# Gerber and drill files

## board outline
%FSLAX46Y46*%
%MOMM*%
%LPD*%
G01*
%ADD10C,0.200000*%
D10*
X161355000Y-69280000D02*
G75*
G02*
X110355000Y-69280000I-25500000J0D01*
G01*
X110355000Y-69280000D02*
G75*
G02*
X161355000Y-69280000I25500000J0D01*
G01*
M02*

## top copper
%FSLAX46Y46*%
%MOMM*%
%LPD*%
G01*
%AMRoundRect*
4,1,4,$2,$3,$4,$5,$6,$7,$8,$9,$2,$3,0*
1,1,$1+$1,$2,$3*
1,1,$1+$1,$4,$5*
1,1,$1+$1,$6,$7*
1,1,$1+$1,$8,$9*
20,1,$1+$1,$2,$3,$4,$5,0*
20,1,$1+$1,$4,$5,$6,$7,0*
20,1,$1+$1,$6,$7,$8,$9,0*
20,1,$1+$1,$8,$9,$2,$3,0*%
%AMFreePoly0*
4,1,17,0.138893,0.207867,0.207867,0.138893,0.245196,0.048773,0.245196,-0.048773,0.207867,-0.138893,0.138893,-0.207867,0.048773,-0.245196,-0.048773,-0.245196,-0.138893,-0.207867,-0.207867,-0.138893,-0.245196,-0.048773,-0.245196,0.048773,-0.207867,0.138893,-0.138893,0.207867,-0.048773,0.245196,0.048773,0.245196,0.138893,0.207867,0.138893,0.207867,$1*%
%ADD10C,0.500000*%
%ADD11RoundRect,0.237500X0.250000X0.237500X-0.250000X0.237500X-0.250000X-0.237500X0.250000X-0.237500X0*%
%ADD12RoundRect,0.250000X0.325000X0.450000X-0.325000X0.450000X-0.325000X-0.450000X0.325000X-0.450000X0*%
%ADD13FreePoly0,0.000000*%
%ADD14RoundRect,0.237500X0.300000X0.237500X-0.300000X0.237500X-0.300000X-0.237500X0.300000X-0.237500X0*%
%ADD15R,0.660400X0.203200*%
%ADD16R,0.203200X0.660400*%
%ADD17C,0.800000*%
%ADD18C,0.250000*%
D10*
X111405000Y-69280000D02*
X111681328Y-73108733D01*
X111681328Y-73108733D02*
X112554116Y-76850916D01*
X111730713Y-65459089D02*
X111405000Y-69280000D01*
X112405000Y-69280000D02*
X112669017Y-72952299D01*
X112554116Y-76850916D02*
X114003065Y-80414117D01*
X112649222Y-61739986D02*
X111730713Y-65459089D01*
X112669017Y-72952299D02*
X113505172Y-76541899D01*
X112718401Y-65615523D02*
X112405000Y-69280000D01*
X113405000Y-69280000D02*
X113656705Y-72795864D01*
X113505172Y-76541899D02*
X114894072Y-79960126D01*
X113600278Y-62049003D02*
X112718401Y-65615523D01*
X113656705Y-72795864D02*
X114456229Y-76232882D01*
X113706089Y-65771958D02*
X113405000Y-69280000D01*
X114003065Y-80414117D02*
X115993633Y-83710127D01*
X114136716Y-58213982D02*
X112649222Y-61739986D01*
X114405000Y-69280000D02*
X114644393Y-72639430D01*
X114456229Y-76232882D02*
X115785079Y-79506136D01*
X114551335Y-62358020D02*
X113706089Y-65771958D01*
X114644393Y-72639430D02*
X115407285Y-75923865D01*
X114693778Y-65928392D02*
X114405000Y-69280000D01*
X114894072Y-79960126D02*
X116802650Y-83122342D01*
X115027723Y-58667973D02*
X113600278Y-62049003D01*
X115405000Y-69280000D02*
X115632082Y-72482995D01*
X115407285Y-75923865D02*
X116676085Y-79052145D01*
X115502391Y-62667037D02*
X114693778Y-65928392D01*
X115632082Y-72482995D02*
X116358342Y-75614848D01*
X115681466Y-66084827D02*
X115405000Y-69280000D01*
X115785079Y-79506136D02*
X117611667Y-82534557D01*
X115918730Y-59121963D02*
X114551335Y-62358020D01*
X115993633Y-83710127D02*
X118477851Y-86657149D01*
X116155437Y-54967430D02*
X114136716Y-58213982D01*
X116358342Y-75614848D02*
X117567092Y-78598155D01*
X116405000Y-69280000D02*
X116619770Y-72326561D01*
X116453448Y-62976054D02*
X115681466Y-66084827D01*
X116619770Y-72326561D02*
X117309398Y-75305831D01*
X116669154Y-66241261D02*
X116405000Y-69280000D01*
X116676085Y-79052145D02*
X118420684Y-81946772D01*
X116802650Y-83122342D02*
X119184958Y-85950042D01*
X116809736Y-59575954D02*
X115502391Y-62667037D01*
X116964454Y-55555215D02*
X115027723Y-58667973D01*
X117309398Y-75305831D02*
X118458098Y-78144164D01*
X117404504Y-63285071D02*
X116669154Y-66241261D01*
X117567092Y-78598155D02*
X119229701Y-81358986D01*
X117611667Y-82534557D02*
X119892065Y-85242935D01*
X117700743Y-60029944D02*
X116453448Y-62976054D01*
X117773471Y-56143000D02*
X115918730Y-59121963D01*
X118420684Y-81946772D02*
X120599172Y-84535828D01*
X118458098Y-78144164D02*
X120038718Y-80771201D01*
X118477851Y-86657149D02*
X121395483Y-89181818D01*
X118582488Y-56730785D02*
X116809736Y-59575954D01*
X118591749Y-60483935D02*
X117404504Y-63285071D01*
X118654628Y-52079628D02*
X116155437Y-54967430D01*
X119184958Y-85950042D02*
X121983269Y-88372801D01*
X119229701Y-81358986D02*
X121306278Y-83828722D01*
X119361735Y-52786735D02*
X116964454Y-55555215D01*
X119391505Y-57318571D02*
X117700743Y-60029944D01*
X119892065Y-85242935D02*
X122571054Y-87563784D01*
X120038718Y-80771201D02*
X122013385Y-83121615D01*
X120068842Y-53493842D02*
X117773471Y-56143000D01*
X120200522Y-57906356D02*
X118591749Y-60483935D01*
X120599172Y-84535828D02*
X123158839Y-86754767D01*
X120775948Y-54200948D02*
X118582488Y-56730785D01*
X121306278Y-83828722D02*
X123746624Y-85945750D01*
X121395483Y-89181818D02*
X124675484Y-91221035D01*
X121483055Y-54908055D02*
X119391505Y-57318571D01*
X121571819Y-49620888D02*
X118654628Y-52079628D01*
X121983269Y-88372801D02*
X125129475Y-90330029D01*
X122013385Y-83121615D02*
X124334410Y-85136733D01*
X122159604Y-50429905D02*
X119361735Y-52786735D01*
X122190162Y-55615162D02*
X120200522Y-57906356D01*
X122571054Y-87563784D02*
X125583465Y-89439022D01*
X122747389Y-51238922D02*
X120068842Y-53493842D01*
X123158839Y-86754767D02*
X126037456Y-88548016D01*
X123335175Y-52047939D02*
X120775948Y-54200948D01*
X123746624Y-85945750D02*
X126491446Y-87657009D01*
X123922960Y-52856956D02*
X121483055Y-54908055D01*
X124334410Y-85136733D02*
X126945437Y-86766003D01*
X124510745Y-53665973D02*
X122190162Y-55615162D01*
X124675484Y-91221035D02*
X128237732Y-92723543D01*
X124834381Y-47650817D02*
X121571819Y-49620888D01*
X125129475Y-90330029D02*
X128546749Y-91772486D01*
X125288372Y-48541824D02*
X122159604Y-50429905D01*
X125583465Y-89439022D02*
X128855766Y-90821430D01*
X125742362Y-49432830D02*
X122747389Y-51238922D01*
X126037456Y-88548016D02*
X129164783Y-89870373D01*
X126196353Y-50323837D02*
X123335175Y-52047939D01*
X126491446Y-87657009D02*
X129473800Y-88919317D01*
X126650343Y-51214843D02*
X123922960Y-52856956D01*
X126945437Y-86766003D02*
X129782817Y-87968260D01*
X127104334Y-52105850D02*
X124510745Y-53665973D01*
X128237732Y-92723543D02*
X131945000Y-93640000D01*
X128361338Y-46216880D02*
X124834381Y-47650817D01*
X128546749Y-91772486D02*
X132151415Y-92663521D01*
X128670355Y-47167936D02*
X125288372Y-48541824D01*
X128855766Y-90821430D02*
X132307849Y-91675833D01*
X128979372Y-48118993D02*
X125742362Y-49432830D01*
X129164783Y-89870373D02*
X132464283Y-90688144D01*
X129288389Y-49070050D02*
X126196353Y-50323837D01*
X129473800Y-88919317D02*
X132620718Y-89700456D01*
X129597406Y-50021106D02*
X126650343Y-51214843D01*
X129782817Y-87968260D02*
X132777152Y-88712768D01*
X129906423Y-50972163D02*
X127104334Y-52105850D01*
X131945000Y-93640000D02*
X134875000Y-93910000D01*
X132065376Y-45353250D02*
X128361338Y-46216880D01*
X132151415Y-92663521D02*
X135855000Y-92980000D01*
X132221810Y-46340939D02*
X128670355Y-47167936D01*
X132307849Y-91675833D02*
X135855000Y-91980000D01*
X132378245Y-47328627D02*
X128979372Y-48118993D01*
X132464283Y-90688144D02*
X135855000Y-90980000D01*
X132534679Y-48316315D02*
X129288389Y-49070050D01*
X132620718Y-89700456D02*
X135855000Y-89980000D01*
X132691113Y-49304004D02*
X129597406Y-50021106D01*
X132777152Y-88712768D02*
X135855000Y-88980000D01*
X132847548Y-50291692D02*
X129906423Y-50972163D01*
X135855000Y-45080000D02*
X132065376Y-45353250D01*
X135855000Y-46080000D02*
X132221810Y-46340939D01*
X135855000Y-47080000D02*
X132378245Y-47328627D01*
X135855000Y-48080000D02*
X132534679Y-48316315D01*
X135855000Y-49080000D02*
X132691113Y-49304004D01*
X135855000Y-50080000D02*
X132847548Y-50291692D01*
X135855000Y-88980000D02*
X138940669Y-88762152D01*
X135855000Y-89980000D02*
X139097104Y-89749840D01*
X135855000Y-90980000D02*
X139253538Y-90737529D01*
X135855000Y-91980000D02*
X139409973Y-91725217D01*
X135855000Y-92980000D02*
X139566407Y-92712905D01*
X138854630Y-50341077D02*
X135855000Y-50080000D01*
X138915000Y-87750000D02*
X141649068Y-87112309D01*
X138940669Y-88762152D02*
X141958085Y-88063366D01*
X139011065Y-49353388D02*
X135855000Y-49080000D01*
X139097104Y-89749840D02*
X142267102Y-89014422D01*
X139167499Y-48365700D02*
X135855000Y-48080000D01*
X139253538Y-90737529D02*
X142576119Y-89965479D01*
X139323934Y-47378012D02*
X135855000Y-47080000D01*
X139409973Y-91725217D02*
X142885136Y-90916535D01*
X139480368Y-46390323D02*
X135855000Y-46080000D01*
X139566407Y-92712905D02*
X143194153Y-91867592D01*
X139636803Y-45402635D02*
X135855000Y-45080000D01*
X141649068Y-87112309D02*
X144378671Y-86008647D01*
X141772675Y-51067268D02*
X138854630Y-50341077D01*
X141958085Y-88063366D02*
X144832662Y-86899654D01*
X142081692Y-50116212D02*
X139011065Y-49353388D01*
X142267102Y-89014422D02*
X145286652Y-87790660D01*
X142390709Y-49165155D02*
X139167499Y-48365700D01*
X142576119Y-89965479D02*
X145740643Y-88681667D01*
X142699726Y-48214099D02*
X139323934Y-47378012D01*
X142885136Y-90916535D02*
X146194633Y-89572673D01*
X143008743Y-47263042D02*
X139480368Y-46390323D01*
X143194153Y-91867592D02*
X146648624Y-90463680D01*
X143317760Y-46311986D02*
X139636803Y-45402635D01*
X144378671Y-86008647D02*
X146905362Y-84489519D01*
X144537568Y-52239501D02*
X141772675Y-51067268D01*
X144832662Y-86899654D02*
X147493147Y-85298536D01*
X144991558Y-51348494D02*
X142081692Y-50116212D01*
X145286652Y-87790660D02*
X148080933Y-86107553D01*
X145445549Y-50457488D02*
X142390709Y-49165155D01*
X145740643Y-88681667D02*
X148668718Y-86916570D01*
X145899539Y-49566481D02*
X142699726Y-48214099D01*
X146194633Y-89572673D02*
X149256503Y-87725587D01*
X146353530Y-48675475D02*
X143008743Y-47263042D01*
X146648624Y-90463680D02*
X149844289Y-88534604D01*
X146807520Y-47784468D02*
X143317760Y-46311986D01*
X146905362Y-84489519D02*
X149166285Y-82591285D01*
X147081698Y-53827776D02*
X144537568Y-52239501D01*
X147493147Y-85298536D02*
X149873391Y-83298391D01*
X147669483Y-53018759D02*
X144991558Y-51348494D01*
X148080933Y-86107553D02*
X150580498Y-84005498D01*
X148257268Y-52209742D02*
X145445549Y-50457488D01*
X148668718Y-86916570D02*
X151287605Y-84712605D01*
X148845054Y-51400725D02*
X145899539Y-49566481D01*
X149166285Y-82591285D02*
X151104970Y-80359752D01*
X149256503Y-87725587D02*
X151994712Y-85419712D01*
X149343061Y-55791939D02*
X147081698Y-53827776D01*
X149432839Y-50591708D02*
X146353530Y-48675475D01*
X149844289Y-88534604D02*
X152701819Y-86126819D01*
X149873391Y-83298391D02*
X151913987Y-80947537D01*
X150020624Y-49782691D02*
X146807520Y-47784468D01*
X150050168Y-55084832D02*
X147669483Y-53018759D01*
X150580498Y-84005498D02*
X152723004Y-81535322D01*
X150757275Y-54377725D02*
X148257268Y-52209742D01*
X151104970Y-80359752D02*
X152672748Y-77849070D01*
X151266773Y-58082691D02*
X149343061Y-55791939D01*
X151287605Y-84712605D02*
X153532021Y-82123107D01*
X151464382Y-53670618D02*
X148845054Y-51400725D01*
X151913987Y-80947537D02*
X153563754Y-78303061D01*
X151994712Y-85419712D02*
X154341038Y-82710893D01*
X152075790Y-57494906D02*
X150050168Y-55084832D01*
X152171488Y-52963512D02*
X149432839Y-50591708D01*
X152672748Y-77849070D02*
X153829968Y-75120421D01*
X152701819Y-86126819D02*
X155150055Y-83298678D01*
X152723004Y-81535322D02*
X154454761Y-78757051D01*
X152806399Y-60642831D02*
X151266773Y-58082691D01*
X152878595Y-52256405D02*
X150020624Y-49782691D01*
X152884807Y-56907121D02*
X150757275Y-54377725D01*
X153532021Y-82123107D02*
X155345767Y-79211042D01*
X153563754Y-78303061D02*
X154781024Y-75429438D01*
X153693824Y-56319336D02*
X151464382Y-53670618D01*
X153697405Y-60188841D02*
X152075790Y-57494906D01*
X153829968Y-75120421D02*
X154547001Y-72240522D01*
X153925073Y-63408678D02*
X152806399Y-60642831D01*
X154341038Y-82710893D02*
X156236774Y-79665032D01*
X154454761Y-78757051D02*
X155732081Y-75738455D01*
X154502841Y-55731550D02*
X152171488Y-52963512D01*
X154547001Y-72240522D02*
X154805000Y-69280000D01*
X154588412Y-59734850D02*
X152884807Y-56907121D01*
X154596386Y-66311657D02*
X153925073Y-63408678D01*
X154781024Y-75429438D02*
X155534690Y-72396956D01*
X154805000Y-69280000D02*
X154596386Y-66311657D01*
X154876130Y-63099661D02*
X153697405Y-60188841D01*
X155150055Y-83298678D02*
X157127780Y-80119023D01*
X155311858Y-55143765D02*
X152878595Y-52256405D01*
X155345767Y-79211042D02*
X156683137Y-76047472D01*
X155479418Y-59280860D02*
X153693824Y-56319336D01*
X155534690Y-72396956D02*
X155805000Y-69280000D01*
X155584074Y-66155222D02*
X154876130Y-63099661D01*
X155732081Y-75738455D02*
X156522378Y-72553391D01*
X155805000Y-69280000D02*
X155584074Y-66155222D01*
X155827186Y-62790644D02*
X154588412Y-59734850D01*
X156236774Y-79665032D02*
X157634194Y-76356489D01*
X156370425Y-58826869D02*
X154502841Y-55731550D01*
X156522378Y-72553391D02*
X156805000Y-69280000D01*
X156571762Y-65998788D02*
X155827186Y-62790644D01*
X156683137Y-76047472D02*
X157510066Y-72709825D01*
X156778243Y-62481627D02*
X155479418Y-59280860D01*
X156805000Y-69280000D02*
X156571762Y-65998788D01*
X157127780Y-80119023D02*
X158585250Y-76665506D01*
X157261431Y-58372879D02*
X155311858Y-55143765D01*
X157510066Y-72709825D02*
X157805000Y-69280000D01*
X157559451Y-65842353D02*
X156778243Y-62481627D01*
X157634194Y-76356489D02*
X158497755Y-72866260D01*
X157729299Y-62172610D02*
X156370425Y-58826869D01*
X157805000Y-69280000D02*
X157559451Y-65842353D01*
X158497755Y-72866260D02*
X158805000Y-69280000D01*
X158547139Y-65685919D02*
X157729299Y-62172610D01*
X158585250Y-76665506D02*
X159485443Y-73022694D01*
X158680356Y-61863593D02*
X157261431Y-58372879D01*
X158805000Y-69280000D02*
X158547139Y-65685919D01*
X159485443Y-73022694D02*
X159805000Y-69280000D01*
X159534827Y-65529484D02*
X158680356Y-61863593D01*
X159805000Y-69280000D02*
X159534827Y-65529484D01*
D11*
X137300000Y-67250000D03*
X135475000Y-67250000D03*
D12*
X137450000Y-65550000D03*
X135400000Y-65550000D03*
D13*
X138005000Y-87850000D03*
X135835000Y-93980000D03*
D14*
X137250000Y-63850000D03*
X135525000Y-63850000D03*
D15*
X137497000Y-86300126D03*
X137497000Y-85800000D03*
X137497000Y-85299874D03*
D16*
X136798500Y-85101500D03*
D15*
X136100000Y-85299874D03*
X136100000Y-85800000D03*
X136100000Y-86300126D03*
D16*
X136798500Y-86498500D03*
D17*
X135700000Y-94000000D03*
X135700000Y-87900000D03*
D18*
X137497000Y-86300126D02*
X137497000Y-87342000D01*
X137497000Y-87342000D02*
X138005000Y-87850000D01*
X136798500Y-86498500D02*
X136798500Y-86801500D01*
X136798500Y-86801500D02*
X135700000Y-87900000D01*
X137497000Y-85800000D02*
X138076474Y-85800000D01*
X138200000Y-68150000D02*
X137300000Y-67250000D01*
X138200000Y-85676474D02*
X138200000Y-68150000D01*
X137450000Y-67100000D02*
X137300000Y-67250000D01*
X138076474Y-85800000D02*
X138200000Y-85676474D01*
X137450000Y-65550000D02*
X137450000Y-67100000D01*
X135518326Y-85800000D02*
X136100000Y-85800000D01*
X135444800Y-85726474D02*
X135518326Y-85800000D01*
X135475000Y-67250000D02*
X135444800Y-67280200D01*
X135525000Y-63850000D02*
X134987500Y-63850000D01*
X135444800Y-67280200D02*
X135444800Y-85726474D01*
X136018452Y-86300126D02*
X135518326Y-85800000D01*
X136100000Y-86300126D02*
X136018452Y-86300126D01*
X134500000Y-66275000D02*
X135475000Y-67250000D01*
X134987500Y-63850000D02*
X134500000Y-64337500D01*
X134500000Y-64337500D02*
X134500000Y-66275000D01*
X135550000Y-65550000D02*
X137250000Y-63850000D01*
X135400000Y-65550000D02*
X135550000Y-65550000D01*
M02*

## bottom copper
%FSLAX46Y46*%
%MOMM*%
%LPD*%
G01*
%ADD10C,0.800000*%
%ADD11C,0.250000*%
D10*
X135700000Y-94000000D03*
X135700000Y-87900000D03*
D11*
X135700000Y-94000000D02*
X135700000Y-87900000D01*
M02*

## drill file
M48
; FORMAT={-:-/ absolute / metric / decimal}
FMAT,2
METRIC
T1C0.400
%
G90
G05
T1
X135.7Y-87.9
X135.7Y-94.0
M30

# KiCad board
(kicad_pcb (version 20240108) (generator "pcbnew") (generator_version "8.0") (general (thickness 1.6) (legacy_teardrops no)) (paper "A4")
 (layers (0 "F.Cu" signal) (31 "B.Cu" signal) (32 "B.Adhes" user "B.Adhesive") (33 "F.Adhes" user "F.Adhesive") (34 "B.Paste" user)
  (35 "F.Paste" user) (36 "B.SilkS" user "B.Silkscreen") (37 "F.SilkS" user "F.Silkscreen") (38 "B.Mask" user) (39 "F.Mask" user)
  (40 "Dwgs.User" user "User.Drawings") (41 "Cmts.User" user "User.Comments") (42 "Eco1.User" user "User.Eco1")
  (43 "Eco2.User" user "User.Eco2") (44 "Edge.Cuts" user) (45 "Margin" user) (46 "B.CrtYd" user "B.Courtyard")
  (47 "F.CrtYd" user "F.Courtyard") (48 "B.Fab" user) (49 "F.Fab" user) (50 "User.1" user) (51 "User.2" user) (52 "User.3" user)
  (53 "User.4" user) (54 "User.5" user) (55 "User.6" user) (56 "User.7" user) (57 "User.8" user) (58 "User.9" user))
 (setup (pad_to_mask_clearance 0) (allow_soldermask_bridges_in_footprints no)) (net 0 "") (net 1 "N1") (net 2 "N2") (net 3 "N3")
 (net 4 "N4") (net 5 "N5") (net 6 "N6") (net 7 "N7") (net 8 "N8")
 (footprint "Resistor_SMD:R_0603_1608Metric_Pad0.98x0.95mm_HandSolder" (layer "F.Cu") (at 136.3875 67.25 180)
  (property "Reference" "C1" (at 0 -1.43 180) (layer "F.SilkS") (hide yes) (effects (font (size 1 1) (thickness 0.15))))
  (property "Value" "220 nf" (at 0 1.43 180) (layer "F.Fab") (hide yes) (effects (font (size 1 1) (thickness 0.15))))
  (pad "1" smd roundrect (at -0.9125 0 180) (size 0.975 0.95) (layers "F.Cu" "F.Paste" "F.Mask") (roundrect_rratio 0.25) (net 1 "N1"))
  (pad "2" smd roundrect (at 0.9125 0 180) (size 0.975 0.95) (layers "F.Cu" "F.Paste" "F.Mask") (roundrect_rratio 0.25) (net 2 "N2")))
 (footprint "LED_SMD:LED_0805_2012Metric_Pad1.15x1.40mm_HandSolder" (layer "F.Cu") (at 136.425 65.55 180)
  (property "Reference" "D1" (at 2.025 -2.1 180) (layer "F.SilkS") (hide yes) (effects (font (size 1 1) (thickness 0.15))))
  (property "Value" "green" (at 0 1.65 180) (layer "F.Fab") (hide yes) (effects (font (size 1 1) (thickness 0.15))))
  (pad "1" smd roundrect (at -1.025 0 180) (size 1.15 1.4) (layers "F.Cu" "F.Paste" "F.Mask") (roundrect_rratio 0.2173913043) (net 1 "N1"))
  (pad "2" smd roundrect (at 1.025 0 180) (size 1.15 1.4) (layers "F.Cu" "F.Paste" "F.Mask") (roundrect_rratio 0.2173913043) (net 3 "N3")))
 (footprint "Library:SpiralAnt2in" (layer "F.Cu") (at 135.855 69.28)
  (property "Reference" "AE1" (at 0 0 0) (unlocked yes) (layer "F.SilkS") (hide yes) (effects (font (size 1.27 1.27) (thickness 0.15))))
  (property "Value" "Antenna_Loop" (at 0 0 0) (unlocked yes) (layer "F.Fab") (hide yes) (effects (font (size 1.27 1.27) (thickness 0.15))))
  (fp_line (start -24.45 0) (end -24.173672 3.828733) (stroke (width 0.5) (type default)) (layer "F.Cu"))
  (fp_line (start -24.173672 3.828733) (end -23.300884 7.570916) (stroke (width 0.5) (type default)) (layer "F.Cu"))
  (fp_line (start -24.124287 -3.820911) (end -24.45 0) (stroke (width 0.5) (type default)) (layer "F.Cu"))
  (fp_line (start -23.45 0) (end -23.185983 3.672299) (stroke (width 0.5) (type default)) (layer "F.Cu"))
  (fp_line (start -23.300884 7.570916) (end -21.851935 11.134117) (stroke (width 0.5) (type default)) (layer "F.Cu"))
  (fp_line (start -23.205778 -7.540014) (end -24.124287 -3.820911) (stroke (width 0.5) (type default)) (layer "F.Cu"))
  (fp_line (start -23.185983 3.672299) (end -22.349828 7.261899) (stroke (width 0.5) (type default)) (layer "F.Cu"))
  (fp_line (start -23.136599 -3.664477) (end -23.45 0) (stroke (width 0.5) (type default)) (layer "F.Cu"))
  (fp_line (start -22.45 0) (end -22.198295 3.515864) (stroke (width 0.5) (type default)) (layer "F.Cu"))
  (fp_line (start -22.349828 7.261899) (end -20.960928 10.680126) (stroke (width 0.5) (type default)) (layer "F.Cu"))
  (fp_line (start -22.254722 -7.230997) (end -23.136599 -3.664477) (stroke (width 0.5) (type default)) (layer "F.Cu"))
  (fp_line (start -22.198295 3.515864) (end -21.398771 6.952882) (stroke (width 0.5) (type default)) (layer "F.Cu"))
  (fp_line (start -22.148911 -3.508042) (end -22.45 0) (stroke (width 0.5) (type default)) (layer "F.Cu"))
  (fp_line (start -21.851935 11.134117) (end -19.861367 14.430127) (stroke (width 0.5) (type default)) (layer "F.Cu"))
  (fp_line (start -21.718284 -11.066018) (end -23.205778 -7.540014) (stroke (width 0.5) (type default)) (layer "F.Cu"))
  (fp_line (start -21.45 0) (end -21.210607 3.35943) (stroke (width 0.5) (type default)) (layer "F.Cu"))
  (fp_line (start -21.398771 6.952882) (end -20.069921 10.226136) (stroke (width 0.5) (type default)) (layer "F.Cu"))
  (fp_line (start -21.303665 -6.92198) (end -22.148911 -3.508042) (stroke (width 0.5) (type default)) (layer "F.Cu"))
  (fp_line (start -21.210607 3.35943) (end -20.447715 6.643865) (stroke (width 0.5) (type default)) (layer "F.Cu"))
  (fp_line (start -21.161222 -3.351608) (end -21.45 0) (stroke (width 0.5) (type default)) (layer "F.Cu"))
  (fp_line (start -20.960928 10.680126) (end -19.05235 13.842342) (stroke (width 0.5) (type default)) (layer "F.Cu"))
  (fp_line (start -20.827277 -10.612027) (end -22.254722 -7.230997) (stroke (width 0.5) (type default)) (layer "F.Cu"))
  (fp_line (start -20.45 0) (end -20.222918 3.202995) (stroke (width 0.5) (type default)) (layer "F.Cu"))
  (fp_line (start -20.447715 6.643865) (end -19.178915 9.772145) (stroke (width 0.5) (type default)) (layer "F.Cu"))
  (fp_line (start -20.352609 -6.612963) (end -21.161222 -3.351608) (stroke (width 0.5) (type default)) (layer "F.Cu"))
  (fp_line (start -20.222918 3.202995) (end -19.496658 6.334848) (stroke (width 0.5) (type default)) (layer "F.Cu"))
  (fp_line (start -20.173534 -3.195173) (end -20.45 0) (stroke (width 0.5) (type default)) (layer "F.Cu"))
  (fp_line (start -20.069921 10.226136) (end -18.243333 13.254557) (stroke (width 0.5) (type default)) (layer "F.Cu"))
  (fp_line (start -19.93627 -10.158037) (end -21.303665 -6.92198) (stroke (width 0.5) (type default)) (layer "F.Cu"))
  (fp_line (start -19.861367 14.430127) (end -17.377149 17.377149) (stroke (width 0.5) (type default)) (layer "F.Cu"))
  (fp_line (start -19.699563 -14.31257) (end -21.718284 -11.066018) (stroke (width 0.5) (type default)) (layer "F.Cu"))
  (fp_line (start -19.496658 6.334848) (end -18.287908 9.318155) (stroke (width 0.5) (type default)) (layer "F.Cu"))
  (fp_line (start -19.45 0) (end -19.23523 3.046561) (stroke (width 0.5) (type default)) (layer "F.Cu"))
  (fp_line (start -19.401552 -6.303946) (end -20.173534 -3.195173) (stroke (width 0.5) (type default)) (layer "F.Cu"))
  (fp_line (start -19.23523 3.046561) (end -18.545602 6.025831) (stroke (width 0.5) (type default)) (layer "F.Cu"))
  (fp_line (start -19.185846 -3.038739) (end -19.45 0) (stroke (width 0.5) (type default)) (layer "F.Cu"))
  (fp_line (start -19.178915 9.772145) (end -17.434316 12.666772) (stroke (width 0.5) (type default)) (layer "F.Cu"))
  (fp_line (start -19.05235 13.842342) (end -16.670042 16.670042) (stroke (width 0.5) (type default)) (layer "F.Cu"))
  (fp_line (start -19.045264 -9.704046) (end -20.352609 -6.612963) (stroke (width 0.5) (type default)) (layer "F.Cu"))
  (fp_line (start -18.890546 -13.724785) (end -20.827277 -10.612027) (stroke (width 0.5) (type default)) (layer "F.Cu"))
  (fp_line (start -18.545602 6.025831) (end -17.396902 8.864164) (stroke (width 0.5) (type default)) (layer "F.Cu"))
  (fp_line (start -18.450496 -5.994929) (end -19.185846 -3.038739) (stroke (width 0.5) (type default)) (layer "F.Cu"))
  (fp_line (start -18.287908 9.318155) (end -16.625299 12.078986) (stroke (width 0.5) (type default)) (layer "F.Cu"))
  (fp_line (start -18.243333 13.254557) (end -15.962935 15.962935) (stroke (width 0.5) (type default)) (layer "F.Cu"))
  (fp_line (start -18.154257 -9.250056) (end -19.401552 -6.303946) (stroke (width 0.5) (type default)) (layer "F.Cu"))
  (fp_line (start -18.081529 -13.137) (end -19.93627 -10.158037) (stroke (width 0.5) (type default)) (layer "F.Cu"))
  (fp_line (start -17.434316 12.666772) (end -15.255828 15.255828) (stroke (width 0.5) (type default)) (layer "F.Cu"))
  (fp_line (start -17.396902 8.864164) (end -15.816282 11.491201) (stroke (width 0.5) (type default)) (layer "F.Cu"))
  (fp_line (start -17.377149 17.377149) (end -14.459517 19.901818) (stroke (width 0.5) (type default)) (layer "F.Cu"))
  (fp_line (start -17.272512 -12.549215) (end -19.045264 -9.704046) (stroke (width 0.5) (type default)) (layer "F.Cu"))
  (fp_line (start -17.263251 -8.796065) (end -18.450496 -5.994929) (stroke (width 0.5) (type default)) (layer "F.Cu"))
  (fp_line (start -17.200372 -17.200372) (end -19.699563 -14.31257) (stroke (width 0.5) (type default)) (layer "F.Cu"))
  (fp_line (start -16.670042 16.670042) (end -13.871731 19.092801) (stroke (width 0.5) (type default)) (layer "F.Cu"))
  (fp_line (start -16.625299 12.078986) (end -14.548722 14.548722) (stroke (width 0.5) (type default)) (layer "F.Cu"))
  (fp_line (start -16.493265 -16.493265) (end -18.890546 -13.724785) (stroke (width 0.5) (type default)) (layer "F.Cu"))
  (fp_line (start -16.463495 -11.961429) (end -18.154257 -9.250056) (stroke (width 0.5) (type default)) (layer "F.Cu"))
  (fp_line (start -15.962935 15.962935) (end -13.283946 18.283784) (stroke (width 0.5) (type default)) (layer "F.Cu"))
  (fp_line (start -15.816282 11.491201) (end -13.841615 13.841615) (stroke (width 0.5) (type default)) (layer "F.Cu"))
  (fp_line (start -15.786158 -15.786158) (end -18.081529 -13.137) (stroke (width 0.5) (type default)) (layer "F.Cu"))
  (fp_line (start -15.654478 -11.373644) (end -17.263251 -8.796065) (stroke (width 0.5) (type default)) (layer "F.Cu"))
  (fp_line (start -15.255828 15.255828) (end -12.696161 17.474767) (stroke (width 0.5) (type default)) (layer "F.Cu"))
  (fp_line (start -15.079052 -15.079052) (end -17.272512 -12.549215) (stroke (width 0.5) (type default)) (layer "F.Cu"))
  (fp_line (start -14.548722 14.548722) (end -12.108376 16.66575) (stroke (width 0.5) (type default)) (layer "F.Cu"))
  (fp_line (start -14.459517 19.901818) (end -11.179516 21.941035) (stroke (width 0.5) (type default)) (layer "F.Cu"))
  (fp_line (start -14.371945 -14.371945) (end -16.463495 -11.961429) (stroke (width 0.5) (type default)) (layer "F.Cu"))
  (fp_line (start -14.283181 -19.659112) (end -17.200372 -17.200372) (stroke (width 0.5) (type default)) (layer "F.Cu"))
  (fp_line (start -13.871731 19.092801) (end -10.725525 21.050029) (stroke (width 0.5) (type default)) (layer "F.Cu"))
  (fp_line (start -13.841615 13.841615) (end -11.52059 15.856733) (stroke (width 0.5) (type default)) (layer "F.Cu"))
  (fp_line (start -13.695396 -18.850095) (end -16.493265 -16.493265) (stroke (width 0.5) (type default)) (layer "F.Cu"))
  (fp_line (start -13.664838 -13.664838) (end -15.654478 -11.373644) (stroke (width 0.5) (type default)) (layer "F.Cu"))
  (fp_line (start -13.283946 18.283784) (end -10.271535 20.159022) (stroke (width 0.5) (type default)) (layer "F.Cu"))
  (fp_line (start -13.107611 -18.041078) (end -15.786158 -15.786158) (stroke (width 0.5) (type default)) (layer "F.Cu"))
  (fp_line (start -12.696161 17.474767) (end -9.817544 19.268016) (stroke (width 0.5) (type default)) (layer "F.Cu"))
  (fp_line (start -12.519825 -17.232061) (end -15.079052 -15.079052) (stroke (width 0.5) (type default)) (layer "F.Cu"))
  (fp_line (start -12.108376 16.66575) (end -9.363554 18.377009) (stroke (width 0.5) (type default)) (layer "F.Cu"))
  (fp_line (start -11.93204 -16.423044) (end -14.371945 -14.371945) (stroke (width 0.5) (type default)) (layer "F.Cu"))
  (fp_line (start -11.52059 15.856733) (end -8.909563 17.486003) (stroke (width 0.5) (type default)) (layer "F.Cu"))
  (fp_line (start -11.344255 -15.614027) (end -13.664838 -13.664838) (stroke (width 0.5) (type default)) (layer "F.Cu"))
  (fp_line (start -11.179516 21.941035) (end -7.617268 23.443543) (stroke (width 0.5) (type default)) (layer "F.Cu"))
  (fp_line (start -11.020619 -21.629183) (end -14.283181 -19.659112) (stroke (width 0.5) (type default)) (layer "F.Cu"))
  (fp_line (start -10.725525 21.050029) (end -7.308251 22.492486) (stroke (width 0.5) (type default)) (layer "F.Cu"))
  (fp_line (start -10.566628 -20.738176) (end -13.695396 -18.850095) (stroke (width 0.5) (type default)) (layer "F.Cu"))
  (fp_line (start -10.271535 20.159022) (end -6.999234 21.54143) (stroke (width 0.5) (type default)) (layer "F.Cu"))
  (fp_line (start -10.112638 -19.84717) (end -13.107611 -18.041078) (stroke (width 0.5) (type default)) (layer "F.Cu"))
  (fp_line (start -9.817544 19.268016) (end -6.690217 20.590373) (stroke (width 0.5) (type default)) (layer "F.Cu"))
  (fp_line (start -9.658647 -18.956163) (end -12.519825 -17.232061) (stroke (width 0.5) (type default)) (layer "F.Cu"))
  (fp_line (start -9.363554 18.377009) (end -6.3812 19.639317) (stroke (width 0.5) (type default)) (layer "F.Cu"))
  (fp_line (start -9.204657 -18.065157) (end -11.93204 -16.423044) (stroke (width 0.5) (type default)) (layer "F.Cu"))
  (fp_line (start -8.909563 17.486003) (end -6.072183 18.68826) (stroke (width 0.5) (type default)) (layer "F.Cu"))
  (fp_line (start -8.750666 -17.17415) (end -11.344255 -15.614027) (stroke (width 0.5) (type default)) (layer "F.Cu"))
  (fp_line (start -7.617268 23.443543) (end -3.91 24.36) (stroke (width 0.5) (type default)) (layer "F.Cu"))
  (fp_line (start -7.493662 -23.06312) (end -11.020619 -21.629183) (stroke (width 0.5) (type default)) (layer "F.Cu"))
  (fp_line (start -7.308251 22.492486) (end -3.703585 23.383521) (stroke (width 0.5) (type default)) (layer "F.Cu"))
  (fp_line (start -7.184645 -22.112064) (end -10.566628 -20.738176) (stroke (width 0.5) (type default)) (layer "F.Cu"))
  (fp_line (start -6.999234 21.54143) (end -3.547151 22.395833) (stroke (width 0.5) (type default)) (layer "F.Cu"))
  (fp_line (start -6.875628 -21.161007) (end -10.112638 -19.84717) (stroke (width 0.5) (type default)) (layer "F.Cu"))
  (fp_line (start -6.690217 20.590373) (end -3.390717 21.408144) (stroke (width 0.5) (type default)) (layer "F.Cu"))
  (fp_line (start -6.566611 -20.20995) (end -9.658647 -18.956163) (stroke (width 0.5) (type default)) (layer "F.Cu"))
  (fp_line (start -6.3812 19.639317) (end -3.234282 20.420456) (stroke (width 0.5) (type default)) (layer "F.Cu"))
  (fp_line (start -6.257594 -19.258894) (end -9.204657 -18.065157) (stroke (width 0.5) (type default)) (layer "F.Cu"))
  (fp_line (start -6.072183 18.68826) (end -3.077848 19.432768) (stroke (width 0.5) (type default)) (layer "F.Cu"))
  (fp_line (start -5.948577 -18.307837) (end -8.750666 -17.17415) (stroke (width 0.5) (type default)) (layer "F.Cu"))
  (fp_line (start -3.91 24.36) (end -0.98 24.63) (stroke (width 0.5) (type default)) (layer "F.Cu"))
  (fp_line (start -3.789624 -23.92675) (end -7.493662 -23.06312) (stroke (width 0.5) (type default)) (layer "F.Cu"))
  (fp_line (start -3.703585 23.383521) (end 0 23.7) (stroke (width 0.5) (type default)) (layer "F.Cu"))
  (fp_line (start -3.63319 -22.939061) (end -7.184645 -22.112064) (stroke (width 0.5) (type default)) (layer "F.Cu"))
  (fp_line (start -3.547151 22.395833) (end 0 22.7) (stroke (width 0.5) (type default)) (layer "F.Cu"))
  (fp_line (start -3.476755 -21.951373) (end -6.875628 -21.161007) (stroke (width 0.5) (type default)) (layer "F.Cu"))
  (fp_line (start -3.390717 21.408144) (end 0 21.7) (stroke (width 0.5) (type default)) (layer "F.Cu"))
  (fp_line (start -3.320321 -20.963685) (end -6.566611 -20.20995) (stroke (width 0.5) (type default)) (layer "F.Cu"))
  (fp_line (start -3.234282 20.420456) (end 0 20.7) (stroke (width 0.5) (type default)) (layer "F.Cu"))
  (fp_line (start -3.163887 -19.975996) (end -6.257594 -19.258894) (stroke (width 0.5) (type default)) (layer "F.Cu"))
  (fp_line (start -3.077848 19.432768) (end 0 19.7) (stroke (width 0.5) (type default)) (layer "F.Cu"))
  (fp_line (start -3.007452 -18.988308) (end -5.948577 -18.307837) (stroke (width 0.5) (type default)) (layer "F.Cu"))
  (fp_line (start 0 -24.2) (end -3.789624 -23.92675) (stroke (width 0.5) (type default)) (layer "F.Cu"))
  (fp_line (start 0 -23.2) (end -3.63319 -22.939061) (stroke (width 0.5) (type default)) (layer "F.Cu"))
  (fp_line (start 0 -22.2) (end -3.476755 -21.951373) (stroke (width 0.5) (type default)) (layer "F.Cu"))
  (fp_line (start 0 -21.2) (end -3.320321 -20.963685) (stroke (width 0.5) (type default)) (layer "F.Cu"))
  (fp_line (start 0 -20.2) (end -3.163887 -19.975996) (stroke (width 0.5) (type default)) (layer "F.Cu"))
  (fp_line (start 0 -19.2) (end -3.007452 -18.988308) (stroke (width 0.5) (type default)) (layer "F.Cu"))
  (fp_line (start 0 19.7) (end 3.085669 19.482152) (stroke (width 0.5) (type default)) (layer "F.Cu"))
  (fp_line (start 0 20.7) (end 3.242104 20.46984) (stroke (width 0.5) (type default)) (layer "F.Cu"))
  (fp_line (start 0 21.7) (end 3.398538 21.457529) (stroke (width 0.5) (type default)) (layer "F.Cu"))
  (fp_line (start 0 22.7) (end 3.554973 22.445217) (stroke (width 0.5) (type default)) (layer "F.Cu"))
  (fp_line (start 0 23.7) (end 3.711407 23.432905) (stroke (width 0.5) (type default)) (layer "F.Cu"))
  (fp_line (start 2.99963 -18.938923) (end 0 -19.2) (stroke (width 0.5) (type default)) (layer "F.Cu"))
  (fp_line (start 3.06 18.47) (end 5.794068 17.832309) (stroke (width 0.5) (type default)) (layer "F.Cu"))
  (fp_line (start 3.085669 19.482152) (end 6.103085 18.783366) (stroke (width 0.5) (type default)) (layer "F.Cu"))
  (fp_line (start 3.156065 -19.926612) (end 0 -20.2) (stroke (width 0.5) (type default)) (layer "F.Cu"))
  (fp_line (start 3.242104 20.46984) (end 6.412102 19.734422) (stroke (width 0.5) (type default)) (layer "F.Cu"))
  (fp_line (start 3.312499 -20.9143) (end 0 -21.2) (stroke (width 0.5) (type default)) (layer "F.Cu"))
  (fp_line (start 3.398538 21.457529) (end 6.721119 20.685479) (stroke (width 0.5) (type default)) (layer "F.Cu"))
  (fp_line (start 3.468934 -21.901988) (end 0 -22.2) (stroke (width 0.5) (type default)) (layer "F.Cu"))
  (fp_line (start 3.554973 22.445217) (end 7.030136 21.636535) (stroke (width 0.5) (type default)) (layer "F.Cu"))
  (fp_line (start 3.625368 -22.889677) (end 0 -23.2) (stroke (width 0.5) (type default)) (layer "F.Cu"))
  (fp_line (start 3.711407 23.432905) (end 7.339153 22.587592) (stroke (width 0.5) (type default)) (layer "F.Cu"))
  (fp_line (start 3.781803 -23.877365) (end 0 -24.2) (stroke (width 0.5) (type default)) (layer "F.Cu"))
  (fp_line (start 5.794068 17.832309) (end 8.523671 16.728647) (stroke (width 0.5) (type default)) (layer "F.Cu"))
  (fp_line (start 5.917675 -18.212732) (end 2.99963 -18.938923) (stroke (width 0.5) (type default)) (layer "F.Cu"))
  (fp_line (start 6.103085 18.783366) (end 8.977662 17.619654) (stroke (width 0.5) (type default)) (layer "F.Cu"))
  (fp_line (start 6.226692 -19.163788) (end 3.156065 -19.926612) (stroke (width 0.5) (type default)) (layer "F.Cu"))
  (fp_line (start 6.412102 19.734422) (end 9.431652 18.51066) (stroke (width 0.5) (type default)) (layer "F.Cu"))
  (fp_line (start 6.535709 -20.114845) (end 3.312499 -20.9143) (stroke (width 0.5) (type default)) (layer "F.Cu"))
  (fp_line (start 6.721119 20.685479) (end 9.885643 19.401667) (stroke (width 0.5) (type default)) (layer "F.Cu"))
  (fp_line (start 6.844726 -21.065901) (end 3.468934 -21.901988) (stroke (width 0.5) (type default)) (layer "F.Cu"))
  (fp_line (start 7.030136 21.636535) (end 10.339633 20.292673) (stroke (width 0.5) (type default)) (layer "F.Cu"))
  (fp_line (start 7.153743 -22.016958) (end 3.625368 -22.889677) (stroke (width 0.5) (type default)) (layer "F.Cu"))
  (fp_line (start 7.339153 22.587592) (end 10.793624 21.18368) (stroke (width 0.5) (type default)) (layer "F.Cu"))
  (fp_line (start 7.46276 -22.968014) (end 3.781803 -23.877365) (stroke (width 0.5) (type default)) (layer "F.Cu"))
  (fp_line (start 8.523671 16.728647) (end 11.050362 15.209519) (stroke (width 0.5) (type default)) (layer "F.Cu"))
  (fp_line (start 8.682568 -17.040499) (end 5.917675 -18.212732) (stroke (width 0.5) (type default)) (layer "F.Cu"))
  (fp_line (start 8.977662 17.619654) (end 11.638147 16.018536) (stroke (width 0.5) (type default)) (layer "F.Cu"))
  (fp_line (start 9.136558 -17.931506) (end 6.226692 -19.163788) (stroke (width 0.5) (type default)) (layer "F.Cu"))
  (fp_line (start 9.431652 18.51066) (end 12.225933 16.827553) (stroke (width 0.5) (type default)) (layer "F.Cu"))
  (fp_line (start 9.590549 -18.822512) (end 6.535709 -20.114845) (stroke (width 0.5) (type default)) (layer "F.Cu"))
  (fp_line (start 9.885643 19.401667) (end 12.813718 17.63657) (stroke (width 0.5) (type default)) (layer "F.Cu"))
  (fp_line (start 10.044539 -19.713519) (end 6.844726 -21.065901) (stroke (width 0.5) (type default)) (layer "F.Cu"))
  (fp_line (start 10.339633 20.292673) (end 13.401503 18.445587) (stroke (width 0.5) (type default)) (layer "F.Cu"))
  (fp_line (start 10.49853 -20.604525) (end 7.153743 -22.016958) (stroke (width 0.5) (type default)) (layer "F.Cu"))
  (fp_line (start 10.793624 21.18368) (end 13.989289 19.254604) (stroke (width 0.5) (type default)) (layer "F.Cu"))
  (fp_line (start 10.95252 -21.495532) (end 7.46276 -22.968014) (stroke (width 0.5) (type default)) (layer "F.Cu"))
  (fp_line (start 11.050362 15.209519) (end 13.311285 13.311285) (stroke (width 0.5) (type default)) (layer "F.Cu"))
  (fp_line (start 11.226698 -15.452224) (end 8.682568 -17.040499) (stroke (width 0.5) (type default)) (layer "F.Cu"))
  (fp_line (start 11.638147 16.018536) (end 14.018391 14.018391) (stroke (width 0.5) (type default)) (layer "F.Cu"))
  (fp_line (start 11.814483 -16.261241) (end 9.136558 -17.931506) (stroke (width 0.5) (type default)) (layer "F.Cu"))
  (fp_line (start 12.225933 16.827553) (end 14.725498 14.725498) (stroke (width 0.5) (type default)) (layer "F.Cu"))
  (fp_line (start 12.402268 -17.070258) (end 9.590549 -18.822512) (stroke (width 0.5) (type default)) (layer "F.Cu"))
  (fp_line (start 12.813718 17.63657) (end 15.432605 15.432605) (stroke (width 0.5) (type default)) (layer "F.Cu"))
  (fp_line (start 12.990054 -17.879275) (end 10.044539 -19.713519) (stroke (width 0.5) (type default)) (layer "F.Cu"))
  (fp_line (start 13.311285 13.311285) (end 15.24997 11.079752) (stroke (width 0.5) (type default)) (layer "F.Cu"))
  (fp_line (start 13.401503 18.445587) (end 16.139712 16.139712) (stroke (width 0.5) (type default)) (layer "F.Cu"))
  (fp_line (start 13.488061 -13.488061) (end 11.226698 -15.452224) (stroke (width 0.5) (type default)) (layer "F.Cu"))
  (fp_line (start 13.577839 -18.688292) (end 10.49853 -20.604525) (stroke (width 0.5) (type default)) (layer "F.Cu"))
  (fp_line (start 13.989289 19.254604) (end 16.846819 16.846819) (stroke (width 0.5) (type default)) (layer "F.Cu"))
  (fp_line (start 14.018391 14.018391) (end 16.058987 11.667537) (stroke (width 0.5) (type default)) (layer "F.Cu"))
  (fp_line (start 14.165624 -19.497309) (end 10.95252 -21.495532) (stroke (width 0.5) (type default)) (layer "F.Cu"))
  (fp_line (start 14.195168 -14.195168) (end 11.814483 -16.261241) (stroke (width 0.5) (type default)) (layer "F.Cu"))
  (fp_line (start 14.725498 14.725498) (end 16.868004 12.255322) (stroke (width 0.5) (type default)) (layer "F.Cu"))
  (fp_line (start 14.902275 -14.902275) (end 12.402268 -17.070258) (stroke (width 0.5) (type default)) (layer "F.Cu"))
  (fp_line (start 15.24997 11.079752) (end 16.817748 8.56907) (stroke (width 0.5) (type default)) (layer "F.Cu"))
  (fp_line (start 15.411773 -11.197309) (end 13.488061 -13.488061) (stroke (width 0.5) (type default)) (layer "F.Cu"))
  (fp_line (start 15.432605 15.432605) (end 17.677021 12.843107) (stroke (width 0.5) (type default)) (layer "F.Cu"))
  (fp_line (start 15.609382 -15.609382) (end 12.990054 -17.879275) (stroke (width 0.5) (type default)) (layer "F.Cu"))
  (fp_line (start 16.058987 11.667537) (end 17.708754 9.023061) (stroke (width 0.5) (type default)) (layer "F.Cu"))
  (fp_line (start 16.139712 16.139712) (end 18.486038 13.430893) (stroke (width 0.5) (type default)) (layer "F.Cu"))
  (fp_line (start 16.22079 -11.785094) (end 14.195168 -14.195168) (stroke (width 0.5) (type default)) (layer "F.Cu"))
  (fp_line (start 16.316488 -16.316488) (end 13.577839 -18.688292) (stroke (width 0.5) (type default)) (layer "F.Cu"))
  (fp_line (start 16.817748 8.56907) (end 17.974968 5.840421) (stroke (width 0.5) (type default)) (layer "F.Cu"))
  (fp_line (start 16.846819 16.846819) (end 19.295055 14.018678) (stroke (width 0.5) (type default)) (layer "F.Cu"))
  (fp_line (start 16.868004 12.255322) (end 18.599761 9.477051) (stroke (width 0.5) (type default)) (layer "F.Cu"))
  (fp_line (start 16.951399 -8.637169) (end 15.411773 -11.197309) (stroke (width 0.5) (type default)) (layer "F.Cu"))
  (fp_line (start 17.023595 -17.023595) (end 14.165624 -19.497309) (stroke (width 0.5) (type default)) (layer "F.Cu"))
  (fp_line (start 17.029807 -12.372879) (end 14.902275 -14.902275) (stroke (width 0.5) (type default)) (layer "F.Cu"))
  (fp_line (start 17.677021 12.843107) (end 19.490767 9.931042) (stroke (width 0.5) (type default)) (layer "F.Cu"))
  (fp_line (start 17.708754 9.023061) (end 18.926024 6.149438) (stroke (width 0.5) (type default)) (layer "F.Cu"))
  (fp_line (start 17.838824 -12.960664) (end 15.609382 -15.609382) (stroke (width 0.5) (type default)) (layer "F.Cu"))
  (fp_line (start 17.842405 -9.091159) (end 16.22079 -11.785094) (stroke (width 0.5) (type default)) (layer "F.Cu"))
  (fp_line (start 17.974968 5.840421) (end 18.692001 2.960522) (stroke (width 0.5) (type default)) (layer "F.Cu"))
  (fp_line (start 18.070073 -5.871322) (end 16.951399 -8.637169) (stroke (width 0.5) (type default)) (layer "F.Cu"))
  (fp_line (start 18.486038 13.430893) (end 20.381774 10.385032) (stroke (width 0.5) (type default)) (layer "F.Cu"))
  (fp_line (start 18.599761 9.477051) (end 19.877081 6.458455) (stroke (width 0.5) (type default)) (layer "F.Cu"))
  (fp_line (start 18.647841 -13.54845) (end 16.316488 -16.316488) (stroke (width 0.5) (type default)) (layer "F.Cu"))
  (fp_line (start 18.692001 2.960522) (end 18.95 0) (stroke (width 0.5) (type default)) (layer "F.Cu"))
  (fp_line (start 18.733412 -9.54515) (end 17.029807 -12.372879) (stroke (width 0.5) (type default)) (layer "F.Cu"))
  (fp_line (start 18.741386 -2.968343) (end 18.070073 -5.871322) (stroke (width 0.5) (type default)) (layer "F.Cu"))
  (fp_line (start 18.926024 6.149438) (end 19.67969 3.116956) (stroke (width 0.5) (type default)) (layer "F.Cu"))
  (fp_line (start 18.95 0) (end 18.741386 -2.968343) (stroke (width 0.5) (type default)) (layer "F.Cu"))
  (fp_line (start 19.02113 -6.180339) (end 17.842405 -9.091159) (stroke (width 0.5) (type default)) (layer "F.Cu"))
  (fp_line (start 19.295055 14.018678) (end 21.27278 10.839023) (stroke (width 0.5) (type default)) (layer "F.Cu"))
  (fp_line (start 19.456858 -14.136235) (end 17.023595 -17.023595) (stroke (width 0.5) (type default)) (layer "F.Cu"))
  (fp_line (start 19.490767 9.931042) (end 20.828137 6.767472) (stroke (width 0.5) (type default)) (layer "F.Cu"))
  (fp_line (start 19.624418 -9.99914) (end 17.838824 -12.960664) (stroke (width 0.5) (type default)) (layer "F.Cu"))
  (fp_line (start 19.67969 3.116956) (end 19.95 0) (stroke (width 0.5) (type default)) (layer "F.Cu"))
  (fp_line (start 19.729074 -3.124778) (end 19.02113 -6.180339) (stroke (width 0.5) (type default)) (layer "F.Cu"))
  (fp_line (start 19.877081 6.458455) (end 20.667378 3.273391) (stroke (width 0.5) (type default)) (layer "F.Cu"))
  (fp_line (start 19.95 0) (end 19.729074 -3.124778) (stroke (width 0.5) (type default)) (layer "F.Cu"))
  (fp_line (start 19.972186 -6.489356) (end 18.733412 -9.54515) (stroke (width 0.5) (type default)) (layer "F.Cu"))
  (fp_line (start 20.381774 10.385032) (end 21.779194 7.076489) (stroke (width 0.5) (type default)) (layer "F.Cu"))
  (fp_line (start 20.515425 -10.453131) (end 18.647841 -13.54845) (stroke (width 0.5) (type default)) (layer "F.Cu"))
  (fp_line (start 20.667378 3.273391) (end 20.95 0) (stroke (width 0.5) (type default)) (layer "F.Cu"))
  (fp_line (start 20.716762 -3.281212) (end 19.972186 -6.489356) (stroke (width 0.5) (type default)) (layer "F.Cu"))
  (fp_line (start 20.828137 6.767472) (end 21.655066 3.429825) (stroke (width 0.5) (type default)) (layer "F.Cu"))
  (fp_line (start 20.923243 -6.798373) (end 19.624418 -9.99914) (stroke (width 0.5) (type default)) (layer "F.Cu"))
  (fp_line (start 20.95 0) (end 20.716762 -3.281212) (stroke (width 0.5) (type default)) (layer "F.Cu"))
  (fp_line (start 21.27278 10.839023) (end 22.73025 7.385506) (stroke (width 0.5) (type default)) (layer "F.Cu"))
  (fp_line (start 21.406431 -10.907121) (end 19.456858 -14.136235) (stroke (width 0.5) (type default)) (layer "F.Cu"))
  (fp_line (start 21.655066 3.429825) (end 21.95 0) (stroke (width 0.5) (type default)) (layer "F.Cu"))
  (fp_line (start 21.704451 -3.437647) (end 20.923243 -6.798373) (stroke (width 0.5) (type default)) (layer "F.Cu"))
  (fp_line (start 21.779194 7.076489) (end 22.642755 3.58626) (stroke (width 0.5) (type default)) (layer "F.Cu"))
  (fp_line (start 21.874299 -7.10739) (end 20.515425 -10.453131) (stroke (width 0.5) (type default)) (layer "F.Cu"))
  (fp_line (start 21.95 0) (end 21.704451 -3.437647) (stroke (width 0.5) (type default)) (layer "F.Cu"))
  (fp_line (start 22.642755 3.58626) (end 22.95 0) (stroke (width 0.5) (type default)) (layer "F.Cu"))
  (fp_line (start 22.692139 -3.594081) (end 21.874299 -7.10739) (stroke (width 0.5) (type default)) (layer "F.Cu"))
  (fp_line (start 22.73025 7.385506) (end 23.630443 3.742694) (stroke (width 0.5) (type default)) (layer "F.Cu"))
  (fp_line (start 22.825356 -7.416407) (end 21.406431 -10.907121) (stroke (width 0.5) (type default)) (layer "F.Cu"))
  (fp_line (start 22.95 0) (end 22.692139 -3.594081) (stroke (width 0.5) (type default)) (layer "F.Cu"))
  (fp_line (start 23.630443 3.742694) (end 23.95 0) (stroke (width 0.5) (type default)) (layer "F.Cu"))
  (fp_line (start 23.679827 -3.750516) (end 22.825356 -7.416407) (stroke (width 0.5) (type default)) (layer "F.Cu"))
  (fp_line (start 23.95 0) (end 23.679827 -3.750516) (stroke (width 0.5) (type default)) (layer "F.Cu"))
  (pad "1" smd custom (at 2.15 18.57) (size 0.5 0.5) (layers "F.Cu") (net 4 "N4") (thermal_bridge_angle 90)
   (options (clearance outline) (anchor circle)) (primitives))
  (pad "2" smd custom (at -0.02 24.7) (size 0.5 0.5) (layers "F.Cu") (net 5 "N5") (thermal_bridge_angle 90)
   (options (clearance outline) (anchor circle)) (primitives)))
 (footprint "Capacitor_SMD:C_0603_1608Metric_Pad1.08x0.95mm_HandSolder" (layer "F.Cu") (at 136.3875 63.85 180)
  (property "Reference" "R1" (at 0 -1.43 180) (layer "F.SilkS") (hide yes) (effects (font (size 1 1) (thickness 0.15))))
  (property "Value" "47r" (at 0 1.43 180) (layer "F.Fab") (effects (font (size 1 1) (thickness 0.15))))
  (pad "1" smd roundrect (at -0.8625 0 180) (size 1.075 0.95) (layers "F.Cu" "F.Paste" "F.Mask") (roundrect_rratio 0.25) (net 3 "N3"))
  (pad "2" smd roundrect (at 0.8625 0 180) (size 1.075 0.95) (layers "F.Cu" "F.Paste" "F.Mask") (roundrect_rratio 0.25) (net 2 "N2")))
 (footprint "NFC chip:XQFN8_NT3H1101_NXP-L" (layer "F.Cu") (at 136.7985 85.8 180)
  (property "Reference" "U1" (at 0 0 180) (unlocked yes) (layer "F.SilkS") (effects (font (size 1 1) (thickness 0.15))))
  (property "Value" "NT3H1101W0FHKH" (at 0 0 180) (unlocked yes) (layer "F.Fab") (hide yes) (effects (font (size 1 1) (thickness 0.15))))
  (pad "1" smd rect (at -0.6985 -0.500126 270) (size 0.2032 0.6604) (layers "F.Cu" "F.Paste" "F.Mask") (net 4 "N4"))
  (pad "2" smd rect (at -0.6985 0 270) (size 0.2032 0.6604) (layers "F.Cu" "F.Paste" "F.Mask") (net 1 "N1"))
  (pad "3" smd rect (at -0.6985 0.500126 270) (size 0.2032 0.6604) (layers "F.Cu" "F.Paste" "F.Mask") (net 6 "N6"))
  (pad "4" smd rect (at 0 0.6985 180) (size 0.2032 0.6604) (layers "F.Cu" "F.Paste" "F.Mask") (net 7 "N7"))
  (pad "5" smd rect (at 0.6985 0.500126 270) (size 0.2032 0.6604) (layers "F.Cu" "F.Paste" "F.Mask") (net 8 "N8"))
  (pad "6" smd rect (at 0.6985 0 270) (size 0.2032 0.6604) (layers "F.Cu" "F.Paste" "F.Mask") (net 2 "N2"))
  (pad "7" smd rect (at 0.6985 -0.500126 270) (size 0.2032 0.6604) (layers "F.Cu" "F.Paste" "F.Mask") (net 2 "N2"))
  (pad "8" smd rect (at 0 -0.6985 180) (size 0.2032 0.6604) (layers "F.Cu" "F.Paste" "F.Mask") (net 5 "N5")))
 (gr_circle (center 135.855 69.28) (end 161.355 69.28) (stroke (width 0.2) (type default)) (fill none) (layer "Edge.Cuts"))
 (segment (start 137.497 86.300126) (end 137.497 87.342) (width 0.25) (layer "F.Cu") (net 4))
 (segment (start 137.497 87.342) (end 138.005 87.85) (width 0.25) (layer "F.Cu") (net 4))
 (segment (start 136.7985 86.4985) (end 136.7985 86.8015) (width 0.25) (layer "F.Cu") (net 5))
 (segment (start 136.7985 86.8015) (end 135.7 87.9) (width 0.25) (layer "F.Cu") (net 5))
 (via (at 135.7 94) (size 0.8) (drill 0.4) (layers "F.Cu" "B.Cu") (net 5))
 (via (at 135.7 87.9) (size 0.8) (drill 0.4) (layers "F.Cu" "B.Cu") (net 5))
 (segment (start 135.7 94) (end 135.7 87.9) (width 0.25) (layer "B.Cu") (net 5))
 (segment (start 137.497 85.8) (end 138.076474 85.8) (width 0.25) (layer "F.Cu") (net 1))
 (segment (start 138.2 68.15) (end 137.3 67.25) (width 0.25) (layer "F.Cu") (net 1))
 (segment (start 138.2 85.676474) (end 138.2 68.15) (width 0.25) (layer "F.Cu") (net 1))
 (segment (start 137.45 67.1) (end 137.3 67.25) (width 0.25) (layer "F.Cu") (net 1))
 (segment (start 138.076474 85.8) (end 138.2 85.676474) (width 0.25) (layer "F.Cu") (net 1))
 (segment (start 137.45 65.55) (end 137.45 67.1) (width 0.25) (layer "F.Cu") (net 1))
 (segment (start 135.518326 85.8) (end 136.1 85.8) (width 0.25) (layer "F.Cu") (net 2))
 (segment (start 135.4448 85.726474) (end 135.518326 85.8) (width 0.25) (layer "F.Cu") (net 2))
 (segment (start 135.475 67.25) (end 135.4448 67.2802) (width 0.25) (layer "F.Cu") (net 2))
 (segment (start 135.525 63.85) (end 134.9875 63.85) (width 0.25) (layer "F.Cu") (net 2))
 (segment (start 135.4448 67.2802) (end 135.4448 85.726474) (width 0.25) (layer "F.Cu") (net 2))
 (segment (start 136.018452 86.300126) (end 135.518326 85.8) (width 0.25) (layer "F.Cu") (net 2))
 (segment (start 136.1 86.300126) (end 136.018452 86.300126) (width 0.25) (layer "F.Cu") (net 2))
 (segment (start 134.5 66.275) (end 135.475 67.25) (width 0.25) (layer "F.Cu") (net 2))
 (segment (start 134.9875 63.85) (end 134.5 64.3375) (width 0.25) (layer "F.Cu") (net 2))
 (segment (start 134.5 64.3375) (end 134.5 66.275) (width 0.25) (layer "F.Cu") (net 2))
 (segment (start 135.55 65.55) (end 137.25 63.85) (width 0.25) (layer "F.Cu") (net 3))
 (segment (start 135.4 65.55) (end 135.55 65.55) (width 0.25) (layer "F.Cu") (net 3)))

